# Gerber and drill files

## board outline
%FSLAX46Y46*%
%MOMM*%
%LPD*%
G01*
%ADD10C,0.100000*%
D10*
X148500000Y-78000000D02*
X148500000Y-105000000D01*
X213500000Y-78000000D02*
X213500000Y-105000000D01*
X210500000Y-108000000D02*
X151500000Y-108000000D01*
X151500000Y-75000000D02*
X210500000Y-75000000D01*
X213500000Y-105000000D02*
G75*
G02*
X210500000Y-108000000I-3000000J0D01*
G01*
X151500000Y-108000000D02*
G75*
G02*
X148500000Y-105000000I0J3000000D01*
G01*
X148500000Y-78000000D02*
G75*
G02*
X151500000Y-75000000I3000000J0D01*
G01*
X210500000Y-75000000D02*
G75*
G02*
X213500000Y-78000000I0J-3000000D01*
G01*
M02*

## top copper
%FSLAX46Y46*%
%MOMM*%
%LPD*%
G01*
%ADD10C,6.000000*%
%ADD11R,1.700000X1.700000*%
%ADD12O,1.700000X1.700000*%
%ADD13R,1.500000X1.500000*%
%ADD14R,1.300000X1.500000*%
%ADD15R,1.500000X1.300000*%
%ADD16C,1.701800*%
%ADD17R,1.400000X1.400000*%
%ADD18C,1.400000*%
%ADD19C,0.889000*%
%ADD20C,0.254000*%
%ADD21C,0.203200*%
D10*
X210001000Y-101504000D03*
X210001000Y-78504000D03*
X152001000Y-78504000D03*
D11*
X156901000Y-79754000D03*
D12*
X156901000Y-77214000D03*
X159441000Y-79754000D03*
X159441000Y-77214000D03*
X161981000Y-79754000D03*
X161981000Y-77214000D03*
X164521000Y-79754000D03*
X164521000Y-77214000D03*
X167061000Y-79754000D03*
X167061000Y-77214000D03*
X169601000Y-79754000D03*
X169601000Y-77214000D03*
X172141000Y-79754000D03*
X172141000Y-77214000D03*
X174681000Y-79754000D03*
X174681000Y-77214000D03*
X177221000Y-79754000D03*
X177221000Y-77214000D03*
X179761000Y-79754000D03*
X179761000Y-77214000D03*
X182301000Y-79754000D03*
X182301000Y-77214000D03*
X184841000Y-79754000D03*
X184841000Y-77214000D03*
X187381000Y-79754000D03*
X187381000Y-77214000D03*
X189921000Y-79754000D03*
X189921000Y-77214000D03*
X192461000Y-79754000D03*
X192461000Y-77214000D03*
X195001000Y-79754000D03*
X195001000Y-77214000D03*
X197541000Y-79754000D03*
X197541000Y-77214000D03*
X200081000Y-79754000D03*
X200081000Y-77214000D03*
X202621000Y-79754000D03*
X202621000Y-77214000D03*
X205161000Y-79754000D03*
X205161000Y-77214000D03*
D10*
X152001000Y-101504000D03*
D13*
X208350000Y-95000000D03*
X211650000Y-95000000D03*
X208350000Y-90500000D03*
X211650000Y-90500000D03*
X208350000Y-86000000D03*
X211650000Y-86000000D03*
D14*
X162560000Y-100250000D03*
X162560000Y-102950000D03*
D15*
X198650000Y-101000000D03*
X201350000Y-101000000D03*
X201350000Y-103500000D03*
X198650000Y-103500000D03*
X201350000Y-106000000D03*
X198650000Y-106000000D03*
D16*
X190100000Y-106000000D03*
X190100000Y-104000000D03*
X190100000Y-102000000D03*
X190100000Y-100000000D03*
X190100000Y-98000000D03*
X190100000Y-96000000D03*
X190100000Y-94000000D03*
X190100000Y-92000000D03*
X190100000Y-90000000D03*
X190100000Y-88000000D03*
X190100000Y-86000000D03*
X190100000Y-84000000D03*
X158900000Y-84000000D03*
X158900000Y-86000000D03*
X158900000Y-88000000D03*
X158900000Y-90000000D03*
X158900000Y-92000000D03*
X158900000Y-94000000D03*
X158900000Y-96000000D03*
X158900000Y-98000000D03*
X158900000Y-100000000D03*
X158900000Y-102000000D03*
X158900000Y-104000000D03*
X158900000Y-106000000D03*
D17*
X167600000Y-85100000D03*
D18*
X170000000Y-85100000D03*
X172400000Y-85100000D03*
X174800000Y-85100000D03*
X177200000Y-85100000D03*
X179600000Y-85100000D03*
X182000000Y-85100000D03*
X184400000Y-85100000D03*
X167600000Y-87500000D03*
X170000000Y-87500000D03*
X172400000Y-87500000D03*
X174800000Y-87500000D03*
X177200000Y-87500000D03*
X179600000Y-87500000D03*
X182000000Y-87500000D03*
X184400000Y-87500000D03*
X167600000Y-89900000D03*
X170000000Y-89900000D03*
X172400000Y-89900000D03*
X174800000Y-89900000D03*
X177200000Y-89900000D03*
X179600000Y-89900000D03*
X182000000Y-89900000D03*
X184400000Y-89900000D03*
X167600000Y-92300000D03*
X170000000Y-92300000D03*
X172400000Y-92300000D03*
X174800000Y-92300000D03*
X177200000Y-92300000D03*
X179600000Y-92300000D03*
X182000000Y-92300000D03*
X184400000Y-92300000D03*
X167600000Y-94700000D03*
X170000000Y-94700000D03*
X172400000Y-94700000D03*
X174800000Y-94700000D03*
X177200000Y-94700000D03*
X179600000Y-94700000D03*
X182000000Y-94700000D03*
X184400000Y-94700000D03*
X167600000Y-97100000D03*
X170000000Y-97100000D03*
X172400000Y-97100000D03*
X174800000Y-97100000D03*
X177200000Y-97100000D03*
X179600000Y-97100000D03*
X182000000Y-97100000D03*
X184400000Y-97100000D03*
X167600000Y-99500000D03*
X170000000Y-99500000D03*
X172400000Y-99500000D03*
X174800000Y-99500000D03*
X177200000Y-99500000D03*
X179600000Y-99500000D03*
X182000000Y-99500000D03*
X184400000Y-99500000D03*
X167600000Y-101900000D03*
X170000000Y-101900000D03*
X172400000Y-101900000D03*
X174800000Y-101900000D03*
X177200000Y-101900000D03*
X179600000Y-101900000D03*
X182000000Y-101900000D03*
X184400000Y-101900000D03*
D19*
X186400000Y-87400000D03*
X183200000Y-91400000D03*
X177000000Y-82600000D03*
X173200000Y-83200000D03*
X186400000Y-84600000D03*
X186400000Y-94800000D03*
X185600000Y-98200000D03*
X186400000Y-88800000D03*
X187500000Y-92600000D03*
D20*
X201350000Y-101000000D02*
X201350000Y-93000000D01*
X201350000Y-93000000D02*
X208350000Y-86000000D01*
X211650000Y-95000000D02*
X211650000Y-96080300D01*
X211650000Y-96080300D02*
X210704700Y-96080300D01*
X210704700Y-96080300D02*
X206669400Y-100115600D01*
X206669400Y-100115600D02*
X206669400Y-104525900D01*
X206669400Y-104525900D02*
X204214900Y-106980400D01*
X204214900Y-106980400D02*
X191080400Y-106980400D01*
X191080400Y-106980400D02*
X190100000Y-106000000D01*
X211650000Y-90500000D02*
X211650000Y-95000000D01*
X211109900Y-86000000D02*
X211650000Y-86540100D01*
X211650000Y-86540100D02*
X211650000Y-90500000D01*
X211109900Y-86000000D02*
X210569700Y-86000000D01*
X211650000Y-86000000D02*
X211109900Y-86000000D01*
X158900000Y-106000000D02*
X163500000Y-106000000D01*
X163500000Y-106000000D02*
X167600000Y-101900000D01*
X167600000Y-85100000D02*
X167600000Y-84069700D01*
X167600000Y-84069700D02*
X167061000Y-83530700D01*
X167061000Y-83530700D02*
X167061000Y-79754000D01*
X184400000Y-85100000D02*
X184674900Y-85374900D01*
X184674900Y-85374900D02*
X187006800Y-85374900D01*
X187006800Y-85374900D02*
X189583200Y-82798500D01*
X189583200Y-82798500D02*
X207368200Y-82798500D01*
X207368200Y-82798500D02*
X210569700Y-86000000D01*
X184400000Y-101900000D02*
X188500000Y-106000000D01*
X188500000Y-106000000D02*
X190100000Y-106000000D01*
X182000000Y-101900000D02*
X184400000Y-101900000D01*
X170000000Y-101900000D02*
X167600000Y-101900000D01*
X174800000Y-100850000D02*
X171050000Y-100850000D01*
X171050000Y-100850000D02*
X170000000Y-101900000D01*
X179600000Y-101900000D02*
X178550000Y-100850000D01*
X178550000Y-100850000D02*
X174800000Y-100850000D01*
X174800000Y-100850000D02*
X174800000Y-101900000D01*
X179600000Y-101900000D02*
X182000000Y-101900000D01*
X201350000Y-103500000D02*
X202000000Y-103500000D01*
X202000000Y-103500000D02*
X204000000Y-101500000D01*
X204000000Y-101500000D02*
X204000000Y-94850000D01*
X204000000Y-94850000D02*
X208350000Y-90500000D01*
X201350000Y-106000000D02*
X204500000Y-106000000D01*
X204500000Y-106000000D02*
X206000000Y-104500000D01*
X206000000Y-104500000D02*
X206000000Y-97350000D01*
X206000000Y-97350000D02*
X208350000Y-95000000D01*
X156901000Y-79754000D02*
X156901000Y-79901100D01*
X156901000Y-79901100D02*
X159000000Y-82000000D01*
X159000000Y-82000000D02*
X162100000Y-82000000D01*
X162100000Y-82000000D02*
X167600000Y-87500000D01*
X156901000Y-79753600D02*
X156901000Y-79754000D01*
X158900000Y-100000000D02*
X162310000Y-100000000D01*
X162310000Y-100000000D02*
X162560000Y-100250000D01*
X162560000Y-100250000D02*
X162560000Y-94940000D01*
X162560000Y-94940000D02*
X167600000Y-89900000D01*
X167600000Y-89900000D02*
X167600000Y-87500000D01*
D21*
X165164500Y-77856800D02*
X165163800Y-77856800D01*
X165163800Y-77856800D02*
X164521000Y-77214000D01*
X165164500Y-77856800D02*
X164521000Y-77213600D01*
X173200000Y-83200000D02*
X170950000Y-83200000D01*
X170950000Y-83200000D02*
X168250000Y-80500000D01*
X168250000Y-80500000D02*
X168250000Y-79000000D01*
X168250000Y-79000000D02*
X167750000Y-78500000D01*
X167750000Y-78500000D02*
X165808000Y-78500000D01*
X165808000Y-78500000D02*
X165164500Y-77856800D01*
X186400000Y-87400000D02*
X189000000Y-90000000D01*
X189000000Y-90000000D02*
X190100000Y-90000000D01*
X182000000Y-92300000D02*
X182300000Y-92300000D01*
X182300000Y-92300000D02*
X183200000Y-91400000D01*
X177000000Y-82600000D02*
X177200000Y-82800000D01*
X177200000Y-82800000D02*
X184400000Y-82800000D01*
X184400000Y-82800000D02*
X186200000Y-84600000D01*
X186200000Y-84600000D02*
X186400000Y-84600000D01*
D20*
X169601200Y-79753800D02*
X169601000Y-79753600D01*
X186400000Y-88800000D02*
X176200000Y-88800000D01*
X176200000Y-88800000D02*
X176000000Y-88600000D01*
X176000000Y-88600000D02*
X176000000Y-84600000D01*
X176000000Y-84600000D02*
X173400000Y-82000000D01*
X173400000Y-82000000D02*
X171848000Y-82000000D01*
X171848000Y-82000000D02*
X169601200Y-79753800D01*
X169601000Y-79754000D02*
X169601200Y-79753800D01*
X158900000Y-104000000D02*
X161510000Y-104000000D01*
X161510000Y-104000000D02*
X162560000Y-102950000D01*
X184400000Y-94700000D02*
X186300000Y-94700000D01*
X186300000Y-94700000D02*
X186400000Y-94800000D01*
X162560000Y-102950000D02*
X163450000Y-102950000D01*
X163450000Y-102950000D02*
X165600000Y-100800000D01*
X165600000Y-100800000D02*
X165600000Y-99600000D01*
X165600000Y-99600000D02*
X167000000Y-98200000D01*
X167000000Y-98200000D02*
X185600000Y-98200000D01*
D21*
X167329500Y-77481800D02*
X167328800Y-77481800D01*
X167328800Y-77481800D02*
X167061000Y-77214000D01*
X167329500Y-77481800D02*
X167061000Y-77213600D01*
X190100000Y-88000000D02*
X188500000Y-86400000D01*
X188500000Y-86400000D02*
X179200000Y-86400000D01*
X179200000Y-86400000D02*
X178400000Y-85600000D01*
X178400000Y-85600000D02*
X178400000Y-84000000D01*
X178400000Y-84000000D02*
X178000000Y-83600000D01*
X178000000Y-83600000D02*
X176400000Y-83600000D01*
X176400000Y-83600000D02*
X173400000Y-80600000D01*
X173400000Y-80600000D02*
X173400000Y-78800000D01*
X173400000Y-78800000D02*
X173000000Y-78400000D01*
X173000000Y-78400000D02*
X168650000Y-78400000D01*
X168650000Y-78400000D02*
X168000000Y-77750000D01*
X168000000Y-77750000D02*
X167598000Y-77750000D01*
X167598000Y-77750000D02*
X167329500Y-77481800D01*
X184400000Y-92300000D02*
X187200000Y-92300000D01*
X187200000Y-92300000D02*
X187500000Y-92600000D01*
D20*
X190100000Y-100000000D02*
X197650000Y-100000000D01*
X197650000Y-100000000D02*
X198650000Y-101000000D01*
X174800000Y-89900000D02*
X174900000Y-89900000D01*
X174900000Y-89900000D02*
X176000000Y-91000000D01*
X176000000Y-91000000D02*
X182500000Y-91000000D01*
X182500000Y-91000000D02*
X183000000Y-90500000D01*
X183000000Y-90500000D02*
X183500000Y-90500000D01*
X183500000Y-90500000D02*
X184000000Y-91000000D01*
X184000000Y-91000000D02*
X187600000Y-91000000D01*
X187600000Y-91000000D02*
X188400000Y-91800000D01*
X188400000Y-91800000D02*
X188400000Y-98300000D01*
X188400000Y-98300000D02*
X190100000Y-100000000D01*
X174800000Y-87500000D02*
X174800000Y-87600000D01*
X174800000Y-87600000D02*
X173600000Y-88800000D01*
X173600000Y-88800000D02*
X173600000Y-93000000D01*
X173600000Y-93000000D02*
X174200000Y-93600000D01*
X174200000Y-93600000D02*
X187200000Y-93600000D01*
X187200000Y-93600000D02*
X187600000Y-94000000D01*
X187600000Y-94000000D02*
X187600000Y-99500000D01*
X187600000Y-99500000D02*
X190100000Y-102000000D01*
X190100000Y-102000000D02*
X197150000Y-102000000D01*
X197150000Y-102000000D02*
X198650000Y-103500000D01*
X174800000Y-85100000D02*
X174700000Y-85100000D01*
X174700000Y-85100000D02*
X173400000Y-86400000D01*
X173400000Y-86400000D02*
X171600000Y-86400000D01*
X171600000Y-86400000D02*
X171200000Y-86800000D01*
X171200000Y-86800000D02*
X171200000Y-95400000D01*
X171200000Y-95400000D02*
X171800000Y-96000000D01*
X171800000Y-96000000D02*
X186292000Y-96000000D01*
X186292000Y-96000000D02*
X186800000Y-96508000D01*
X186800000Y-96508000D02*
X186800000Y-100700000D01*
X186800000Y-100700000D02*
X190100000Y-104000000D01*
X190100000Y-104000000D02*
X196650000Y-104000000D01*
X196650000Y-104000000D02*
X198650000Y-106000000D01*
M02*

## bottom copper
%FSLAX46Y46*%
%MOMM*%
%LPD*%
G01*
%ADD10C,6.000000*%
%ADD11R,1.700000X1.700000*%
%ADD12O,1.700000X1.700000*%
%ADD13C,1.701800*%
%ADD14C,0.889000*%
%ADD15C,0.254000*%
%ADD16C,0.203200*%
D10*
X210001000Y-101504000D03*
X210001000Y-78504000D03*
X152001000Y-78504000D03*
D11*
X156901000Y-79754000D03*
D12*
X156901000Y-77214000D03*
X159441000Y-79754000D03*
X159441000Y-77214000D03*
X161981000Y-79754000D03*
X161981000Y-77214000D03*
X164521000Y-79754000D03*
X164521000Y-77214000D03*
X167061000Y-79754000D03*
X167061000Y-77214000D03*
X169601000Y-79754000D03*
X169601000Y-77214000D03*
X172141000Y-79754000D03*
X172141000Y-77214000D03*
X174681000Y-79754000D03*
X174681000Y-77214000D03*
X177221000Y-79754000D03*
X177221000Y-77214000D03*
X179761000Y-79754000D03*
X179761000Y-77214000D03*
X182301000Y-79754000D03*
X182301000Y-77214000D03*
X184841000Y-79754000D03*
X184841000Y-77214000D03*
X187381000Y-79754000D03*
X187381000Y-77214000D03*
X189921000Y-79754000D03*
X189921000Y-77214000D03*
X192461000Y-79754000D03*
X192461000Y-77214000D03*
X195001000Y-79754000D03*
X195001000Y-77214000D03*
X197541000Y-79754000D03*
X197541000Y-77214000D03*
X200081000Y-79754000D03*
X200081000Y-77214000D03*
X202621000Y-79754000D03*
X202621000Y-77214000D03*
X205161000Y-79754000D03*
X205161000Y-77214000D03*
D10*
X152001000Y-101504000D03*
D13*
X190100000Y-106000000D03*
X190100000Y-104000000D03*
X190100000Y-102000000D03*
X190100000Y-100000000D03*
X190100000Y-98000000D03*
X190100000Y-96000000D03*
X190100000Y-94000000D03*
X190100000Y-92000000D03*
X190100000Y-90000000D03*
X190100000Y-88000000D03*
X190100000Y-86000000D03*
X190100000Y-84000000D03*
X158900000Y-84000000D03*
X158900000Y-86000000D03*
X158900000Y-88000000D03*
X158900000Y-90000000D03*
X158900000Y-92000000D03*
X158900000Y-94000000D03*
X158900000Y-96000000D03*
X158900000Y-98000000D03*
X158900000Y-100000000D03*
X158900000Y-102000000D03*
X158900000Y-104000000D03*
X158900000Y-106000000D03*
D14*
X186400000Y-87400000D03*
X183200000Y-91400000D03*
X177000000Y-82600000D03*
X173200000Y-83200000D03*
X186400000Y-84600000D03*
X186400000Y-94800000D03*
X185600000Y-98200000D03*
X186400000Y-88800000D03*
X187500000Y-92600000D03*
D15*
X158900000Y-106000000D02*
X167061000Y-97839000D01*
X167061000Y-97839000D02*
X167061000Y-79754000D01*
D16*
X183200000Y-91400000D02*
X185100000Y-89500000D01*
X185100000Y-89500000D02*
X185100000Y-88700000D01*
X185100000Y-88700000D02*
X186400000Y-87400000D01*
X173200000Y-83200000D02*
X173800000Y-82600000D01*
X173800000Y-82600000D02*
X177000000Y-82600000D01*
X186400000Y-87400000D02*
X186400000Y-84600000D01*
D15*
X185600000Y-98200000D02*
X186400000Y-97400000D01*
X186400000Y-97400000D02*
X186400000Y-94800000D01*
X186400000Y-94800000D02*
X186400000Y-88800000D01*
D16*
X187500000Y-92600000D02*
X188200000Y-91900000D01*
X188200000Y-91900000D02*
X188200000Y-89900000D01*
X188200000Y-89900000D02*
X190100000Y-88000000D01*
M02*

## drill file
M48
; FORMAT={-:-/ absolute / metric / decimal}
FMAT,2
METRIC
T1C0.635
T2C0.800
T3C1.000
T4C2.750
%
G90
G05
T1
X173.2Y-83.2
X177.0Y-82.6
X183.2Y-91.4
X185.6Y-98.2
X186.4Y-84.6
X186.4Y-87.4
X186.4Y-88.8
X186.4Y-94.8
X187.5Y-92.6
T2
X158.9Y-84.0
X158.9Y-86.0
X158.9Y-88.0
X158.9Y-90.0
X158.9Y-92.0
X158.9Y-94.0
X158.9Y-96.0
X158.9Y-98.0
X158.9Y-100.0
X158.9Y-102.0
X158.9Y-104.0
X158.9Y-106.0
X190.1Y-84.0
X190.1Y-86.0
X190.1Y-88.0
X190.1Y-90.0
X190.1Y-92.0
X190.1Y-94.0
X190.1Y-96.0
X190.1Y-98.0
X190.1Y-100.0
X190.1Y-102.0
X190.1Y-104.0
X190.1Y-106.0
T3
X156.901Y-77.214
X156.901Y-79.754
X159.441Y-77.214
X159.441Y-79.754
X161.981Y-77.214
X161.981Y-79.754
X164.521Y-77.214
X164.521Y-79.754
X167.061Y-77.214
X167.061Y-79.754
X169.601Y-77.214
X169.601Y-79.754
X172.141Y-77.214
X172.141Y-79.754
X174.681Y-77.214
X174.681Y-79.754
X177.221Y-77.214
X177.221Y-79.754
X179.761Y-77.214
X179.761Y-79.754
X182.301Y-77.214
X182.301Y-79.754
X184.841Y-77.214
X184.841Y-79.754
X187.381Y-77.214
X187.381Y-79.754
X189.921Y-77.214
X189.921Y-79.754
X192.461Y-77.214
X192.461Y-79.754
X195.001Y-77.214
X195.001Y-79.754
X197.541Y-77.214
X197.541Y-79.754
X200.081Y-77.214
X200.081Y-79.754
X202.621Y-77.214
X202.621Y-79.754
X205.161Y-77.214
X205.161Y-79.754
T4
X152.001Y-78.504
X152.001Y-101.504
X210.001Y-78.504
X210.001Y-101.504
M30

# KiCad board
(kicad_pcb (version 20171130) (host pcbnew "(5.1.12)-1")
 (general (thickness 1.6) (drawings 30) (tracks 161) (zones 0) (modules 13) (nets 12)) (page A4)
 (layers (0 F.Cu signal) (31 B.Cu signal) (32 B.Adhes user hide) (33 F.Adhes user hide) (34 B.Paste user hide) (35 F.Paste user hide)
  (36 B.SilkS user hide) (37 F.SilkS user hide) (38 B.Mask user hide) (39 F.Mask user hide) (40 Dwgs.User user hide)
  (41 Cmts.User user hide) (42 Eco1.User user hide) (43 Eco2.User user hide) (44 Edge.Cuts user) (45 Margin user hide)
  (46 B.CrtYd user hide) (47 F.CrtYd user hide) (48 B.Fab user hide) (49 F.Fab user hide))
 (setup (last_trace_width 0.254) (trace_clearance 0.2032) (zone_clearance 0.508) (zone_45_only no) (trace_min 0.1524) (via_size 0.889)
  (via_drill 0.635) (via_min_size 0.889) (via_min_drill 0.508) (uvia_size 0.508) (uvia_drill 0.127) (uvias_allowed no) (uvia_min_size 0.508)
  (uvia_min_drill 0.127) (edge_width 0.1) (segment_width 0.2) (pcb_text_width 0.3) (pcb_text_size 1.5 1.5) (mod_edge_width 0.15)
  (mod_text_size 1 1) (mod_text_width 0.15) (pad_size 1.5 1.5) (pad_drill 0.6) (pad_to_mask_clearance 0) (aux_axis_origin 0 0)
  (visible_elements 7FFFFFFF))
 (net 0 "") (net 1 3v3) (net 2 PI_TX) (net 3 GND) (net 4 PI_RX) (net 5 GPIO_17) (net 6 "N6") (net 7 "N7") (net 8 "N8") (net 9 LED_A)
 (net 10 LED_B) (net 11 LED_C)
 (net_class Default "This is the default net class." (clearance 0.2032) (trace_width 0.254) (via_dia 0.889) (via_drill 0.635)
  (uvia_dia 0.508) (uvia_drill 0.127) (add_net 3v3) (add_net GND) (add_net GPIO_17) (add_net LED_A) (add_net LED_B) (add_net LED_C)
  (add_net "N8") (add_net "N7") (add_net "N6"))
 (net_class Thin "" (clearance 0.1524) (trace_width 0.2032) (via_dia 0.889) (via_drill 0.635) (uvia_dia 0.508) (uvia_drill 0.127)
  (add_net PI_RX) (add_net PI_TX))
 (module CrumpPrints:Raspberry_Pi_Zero (layer F.Cu) (at 148.501 105.004)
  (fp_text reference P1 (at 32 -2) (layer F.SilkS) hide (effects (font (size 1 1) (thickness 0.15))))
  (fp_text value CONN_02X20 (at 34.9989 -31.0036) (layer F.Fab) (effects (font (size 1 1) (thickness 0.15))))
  (pad "" np_thru_hole circle (at 61.5 -3.5) (size 6 6) (drill 2.75) (layers *.Cu *.Mask F.SilkS))
  (pad "" np_thru_hole circle (at 61.5 -26.5) (size 6 6) (drill 2.75) (layers *.Cu *.Mask F.SilkS))
  (pad "" np_thru_hole circle (at 3.5 -26.5) (size 6 6) (drill 2.75) (layers *.Cu *.Mask F.SilkS))
  (pad 1 thru_hole rect (at 8.4 -25.25 90) (size 1.7 1.7) (drill 1) (layers *.Cu *.Mask) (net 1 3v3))
  (pad 2 thru_hole oval (at 8.4 -27.79 90) (size 1.7 1.7) (drill 1) (layers *.Cu *.Mask))
  (pad 3 thru_hole oval (at 10.94 -25.25 90) (size 1.7 1.7) (drill 1) (layers *.Cu *.Mask))
  (pad 4 thru_hole oval (at 10.94 -27.79 90) (size 1.7 1.7) (drill 1) (layers *.Cu *.Mask))
  (pad 5 thru_hole oval (at 13.48 -25.25 90) (size 1.7 1.7) (drill 1) (layers *.Cu *.Mask))
  (pad 6 thru_hole oval (at 13.48 -27.79 90) (size 1.7 1.7) (drill 1) (layers *.Cu *.Mask))
  (pad 7 thru_hole oval (at 16.02 -25.25 90) (size 1.7 1.7) (drill 1) (layers *.Cu *.Mask))
  (pad 8 thru_hole oval (at 16.02 -27.79 90) (size 1.7 1.7) (drill 1) (layers *.Cu *.Mask) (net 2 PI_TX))
  (pad 9 thru_hole oval (at 18.56 -25.25 90) (size 1.7 1.7) (drill 1) (layers *.Cu *.Mask) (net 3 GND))
  (pad 10 thru_hole oval (at 18.56 -27.79 90) (size 1.7 1.7) (drill 1) (layers *.Cu *.Mask) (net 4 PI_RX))
  (pad 11 thru_hole oval (at 21.1 -25.25 90) (size 1.7 1.7) (drill 1) (layers *.Cu *.Mask) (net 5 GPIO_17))
  (pad 12 thru_hole oval (at 21.1 -27.79 90) (size 1.7 1.7) (drill 1) (layers *.Cu *.Mask))
  (pad 13 thru_hole oval (at 23.64 -25.25 90) (size 1.7 1.7) (drill 1) (layers *.Cu *.Mask))
  (pad 14 thru_hole oval (at 23.64 -27.79 90) (size 1.7 1.7) (drill 1) (layers *.Cu *.Mask))
  (pad 15 thru_hole oval (at 26.18 -25.25 90) (size 1.7 1.7) (drill 1) (layers *.Cu *.Mask))
  (pad 16 thru_hole oval (at 26.18 -27.79 90) (size 1.7 1.7) (drill 1) (layers *.Cu *.Mask))
  (pad 17 thru_hole oval (at 28.72 -25.25 90) (size 1.7 1.7) (drill 1) (layers *.Cu *.Mask))
  (pad 18 thru_hole oval (at 28.72 -27.79 90) (size 1.7 1.7) (drill 1) (layers *.Cu *.Mask))
  (pad 19 thru_hole oval (at 31.26 -25.25 90) (size 1.7 1.7) (drill 1) (layers *.Cu *.Mask))
  (pad 20 thru_hole oval (at 31.26 -27.79 90) (size 1.7 1.7) (drill 1) (layers *.Cu *.Mask))
  (pad 21 thru_hole oval (at 33.8 -25.25 90) (size 1.7 1.7) (drill 1) (layers *.Cu *.Mask))
  (pad 22 thru_hole oval (at 33.8 -27.79 90) (size 1.7 1.7) (drill 1) (layers *.Cu *.Mask))
  (pad 23 thru_hole oval (at 36.34 -25.25 90) (size 1.7 1.7) (drill 1) (layers *.Cu *.Mask))
  (pad 24 thru_hole oval (at 36.34 -27.79 90) (size 1.7 1.7) (drill 1) (layers *.Cu *.Mask))
  (pad 25 thru_hole oval (at 38.88 -25.25 90) (size 1.7 1.7) (drill 1) (layers *.Cu *.Mask))
  (pad 26 thru_hole oval (at 38.88 -27.79 90) (size 1.7 1.7) (drill 1) (layers *.Cu *.Mask))
  (pad 27 thru_hole oval (at 41.42 -25.25 90) (size 1.7 1.7) (drill 1) (layers *.Cu *.Mask))
  (pad 28 thru_hole oval (at 41.42 -27.79 90) (size 1.7 1.7) (drill 1) (layers *.Cu *.Mask))
  (pad 29 thru_hole oval (at 43.96 -25.25 90) (size 1.7 1.7) (drill 1) (layers *.Cu *.Mask))
  (pad 30 thru_hole oval (at 43.96 -27.79 90) (size 1.7 1.7) (drill 1) (layers *.Cu *.Mask))
  (pad 31 thru_hole oval (at 46.5 -25.25 90) (size 1.7 1.7) (drill 1) (layers *.Cu *.Mask))
  (pad 32 thru_hole oval (at 46.5 -27.79 90) (size 1.7 1.7) (drill 1) (layers *.Cu *.Mask))
  (pad 33 thru_hole oval (at 49.04 -25.25 90) (size 1.7 1.7) (drill 1) (layers *.Cu *.Mask))
  (pad 34 thru_hole oval (at 49.04 -27.79 90) (size 1.7 1.7) (drill 1) (layers *.Cu *.Mask))
  (pad 35 thru_hole oval (at 51.58 -25.25 90) (size 1.7 1.7) (drill 1) (layers *.Cu *.Mask))
  (pad 36 thru_hole oval (at 51.58 -27.79 90) (size 1.7 1.7) (drill 1) (layers *.Cu *.Mask))
  (pad 37 thru_hole oval (at 54.12 -25.25 90) (size 1.7 1.7) (drill 1) (layers *.Cu *.Mask))
  (pad 38 thru_hole oval (at 54.12 -27.79 90) (size 1.7 1.7) (drill 1) (layers *.Cu *.Mask))
  (pad 39 thru_hole oval (at 56.66 -25.25 90) (size 1.7 1.7) (drill 1) (layers *.Cu *.Mask))
  (pad 40 thru_hole oval (at 56.66 -27.79 90) (size 1.7 1.7) (drill 1) (layers *.Cu *.Mask))
  (pad "" np_thru_hole circle (at 3.5 -3.5) (size 6 6) (drill 2.75) (layers *.Cu *.Mask F.SilkS)))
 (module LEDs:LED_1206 (layer F.Cu) (at 210 95 180)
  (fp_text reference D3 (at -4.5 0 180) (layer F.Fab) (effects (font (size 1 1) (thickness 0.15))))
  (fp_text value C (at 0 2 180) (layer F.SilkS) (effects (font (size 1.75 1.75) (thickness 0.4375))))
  (pad 2 smd rect (at 1.65 0) (size 1.5 1.5) (layers F.Cu F.Paste F.Mask) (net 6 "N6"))
  (pad 1 smd rect (at -1.65 0) (size 1.5 1.5) (layers F.Cu F.Paste F.Mask) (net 3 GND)))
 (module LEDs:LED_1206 (layer F.Cu) (at 210 90.5 180)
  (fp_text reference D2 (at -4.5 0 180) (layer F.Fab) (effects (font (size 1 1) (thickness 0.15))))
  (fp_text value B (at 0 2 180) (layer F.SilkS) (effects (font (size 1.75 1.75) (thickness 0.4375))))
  (pad 2 smd rect (at 1.65 0) (size 1.5 1.5) (layers F.Cu F.Paste F.Mask) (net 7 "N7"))
  (pad 1 smd rect (at -1.65 0) (size 1.5 1.5) (layers F.Cu F.Paste F.Mask) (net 3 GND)))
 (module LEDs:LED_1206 (layer F.Cu) (at 210 86 180)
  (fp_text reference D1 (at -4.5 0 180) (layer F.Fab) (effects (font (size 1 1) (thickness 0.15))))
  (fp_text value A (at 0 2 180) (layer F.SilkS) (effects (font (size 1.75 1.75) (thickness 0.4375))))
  (pad 2 smd rect (at 1.65 0) (size 1.5 1.5) (layers F.Cu F.Paste F.Mask) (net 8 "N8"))
  (pad 1 smd rect (at -1.65 0) (size 1.5 1.5) (layers F.Cu F.Paste F.Mask) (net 3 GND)))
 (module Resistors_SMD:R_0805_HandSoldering (layer F.Cu) (at 162.56 101.6 270)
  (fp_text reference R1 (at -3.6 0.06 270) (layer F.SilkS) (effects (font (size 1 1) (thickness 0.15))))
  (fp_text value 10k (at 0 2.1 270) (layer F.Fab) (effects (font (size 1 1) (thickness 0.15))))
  (pad 1 smd rect (at -1.35 0 270) (size 1.5 1.3) (layers F.Cu F.Paste F.Mask) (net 1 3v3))
  (pad 2 smd rect (at 1.35 0 270) (size 1.5 1.3) (layers F.Cu F.Paste F.Mask) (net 5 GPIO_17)))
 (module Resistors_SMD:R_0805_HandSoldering (layer F.Cu) (at 200 101)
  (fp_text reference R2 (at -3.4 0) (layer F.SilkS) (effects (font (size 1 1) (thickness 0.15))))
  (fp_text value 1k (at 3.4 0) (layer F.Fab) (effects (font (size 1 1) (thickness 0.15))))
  (pad 1 smd rect (at -1.35 0) (size 1.5 1.3) (layers F.Cu F.Paste F.Mask) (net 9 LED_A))
  (pad 2 smd rect (at 1.35 0) (size 1.5 1.3) (layers F.Cu F.Paste F.Mask) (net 8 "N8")))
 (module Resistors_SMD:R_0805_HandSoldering (layer F.Cu) (at 200 103.5 180)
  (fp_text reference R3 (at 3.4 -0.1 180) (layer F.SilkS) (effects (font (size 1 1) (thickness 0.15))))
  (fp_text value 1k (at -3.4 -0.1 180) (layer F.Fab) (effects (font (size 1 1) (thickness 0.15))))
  (pad 1 smd rect (at -1.35 0 180) (size 1.5 1.3) (layers F.Cu F.Paste F.Mask) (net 7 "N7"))
  (pad 2 smd rect (at 1.35 0 180) (size 1.5 1.3) (layers F.Cu F.Paste F.Mask) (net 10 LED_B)))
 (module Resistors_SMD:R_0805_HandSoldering (layer F.Cu) (at 200 106 180)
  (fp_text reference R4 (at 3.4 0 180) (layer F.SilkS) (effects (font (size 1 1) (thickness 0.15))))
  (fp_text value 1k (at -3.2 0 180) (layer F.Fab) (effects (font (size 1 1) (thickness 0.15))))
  (pad 1 smd rect (at -1.35 0 180) (size 1.5 1.3) (layers F.Cu F.Paste F.Mask) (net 6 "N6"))
  (pad 2 smd rect (at 1.35 0 180) (size 1.5 1.3) (layers F.Cu F.Paste F.Mask) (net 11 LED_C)))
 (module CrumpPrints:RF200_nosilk (layer F.Cu) (at 174.5 95 180)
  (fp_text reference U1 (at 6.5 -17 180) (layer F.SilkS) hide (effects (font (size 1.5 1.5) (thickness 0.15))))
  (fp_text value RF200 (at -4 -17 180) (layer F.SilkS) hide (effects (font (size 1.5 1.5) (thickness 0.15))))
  (pad 1 thru_hole circle (at -15.6 -11 180) (size 1.7018 1.7018) (drill 0.800001) (layers *.Cu *.Mask) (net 3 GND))
  (pad 2 thru_hole circle (at -15.6 -9 180) (size 1.7018 1.7018) (drill 0.800001) (layers *.Cu *.Mask) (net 11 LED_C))
  (pad 3 thru_hole circle (at -15.6 -7 180) (size 1.7018 1.7018) (drill 0.800001) (layers *.Cu *.Mask) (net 10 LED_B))
  (pad 4 thru_hole circle (at -15.6 -5 180) (size 1.7018 1.7018) (drill 0.800001) (layers *.Cu *.Mask) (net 9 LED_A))
  (pad 5 thru_hole circle (at -15.6 -3 180) (size 1.7018 1.7018) (drill 0.800001) (layers *.Cu *.Mask))
  (pad 6 thru_hole circle (at -15.6 -1 180) (size 1.7018 1.7018) (drill 0.800001) (layers *.Cu *.Mask))
  (pad 7 thru_hole circle (at -15.6 1 180) (size 1.7018 1.7018) (drill 0.800001) (layers *.Cu *.Mask))
  (pad 8 thru_hole circle (at -15.6 3 180) (size 1.7018 1.7018) (drill 0.800001) (layers *.Cu *.Mask))
  (pad 9 thru_hole circle (at -15.6 5 180) (size 1.7018 1.7018) (drill 0.800001) (layers *.Cu *.Mask) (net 2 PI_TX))
  (pad 10 thru_hole circle (at -15.6 7 180) (size 1.7018 1.7018) (drill 0.800001) (layers *.Cu *.Mask) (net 4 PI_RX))
  (pad 11 thru_hole circle (at -15.6 9 180) (size 1.7018 1.7018) (drill 0.800001) (layers *.Cu *.Mask))
  (pad 12 thru_hole circle (at -15.6 11 180) (size 1.7018 1.7018) (drill 0.800001) (layers *.Cu *.Mask))
  (pad 13 thru_hole circle (at 15.6 11 180) (size 1.7018 1.7018) (drill 0.800001) (layers *.Cu *.Mask))
  (pad 14 thru_hole circle (at 15.6 9 180) (size 1.7018 1.7018) (drill 0.800001) (layers *.Cu *.Mask))
  (pad 15 thru_hole circle (at 15.6 7 180) (size 1.7018 1.7018) (drill 0.800001) (layers *.Cu *.Mask))
  (pad 16 thru_hole circle (at 15.6 5 180) (size 1.7018 1.7018) (drill 0.800001) (layers *.Cu *.Mask))
  (pad 17 thru_hole circle (at 15.6 3 180) (size 1.7018 1.7018) (drill 0.800001) (layers *.Cu *.Mask))
  (pad 18 thru_hole circle (at 15.6 1 180) (size 1.7018 1.7018) (drill 0.800001) (layers *.Cu *.Mask))
  (pad 19 thru_hole circle (at 15.6 -1 180) (size 1.7018 1.7018) (drill 0.800001) (layers *.Cu *.Mask))
  (pad 20 thru_hole circle (at 15.6 -3 180) (size 1.7018 1.7018) (drill 0.800001) (layers *.Cu *.Mask))
  (pad 21 thru_hole circle (at 15.6 -5 180) (size 1.7018 1.7018) (drill 0.800001) (layers *.Cu *.Mask) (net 1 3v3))
  (pad 22 thru_hole circle (at 15.6 -7 180) (size 1.7018 1.7018) (drill 0.800001) (layers *.Cu *.Mask))
  (pad 23 thru_hole circle (at 15.6 -9 180) (size 1.7018 1.7018) (drill 0.800001) (layers *.Cu *.Mask) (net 5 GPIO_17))
  (pad 24 thru_hole circle (at 15.6 -11 180) (size 1.7018 1.7018) (drill 0.800001) (layers *.Cu *.Mask) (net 3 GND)))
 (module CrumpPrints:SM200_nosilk (layer F.Cu) (at 176 93.5 180)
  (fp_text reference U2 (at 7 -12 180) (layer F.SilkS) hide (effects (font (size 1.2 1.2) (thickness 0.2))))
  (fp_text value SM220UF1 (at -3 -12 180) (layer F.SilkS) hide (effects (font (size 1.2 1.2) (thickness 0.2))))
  (pad A1 smd rect (at 8.4 8.4 270) (size 1.4 1.4) (layers F.Cu F.Paste F.Mask) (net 3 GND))
  (pad B1 smd circle (at 6 8.4 270) (size 1.4 1.4) (layers F.Cu F.Paste F.Mask))
  (pad C1 smd circle (at 3.6 8.4 270) (size 1.4 1.4) (layers F.Cu F.Paste F.Mask))
  (pad D1 smd circle (at 1.2 8.4 270) (size 1.4 1.4) (layers F.Cu F.Paste F.Mask) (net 11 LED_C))
  (pad E1 smd circle (at -1.2 8.4 270) (size 1.4 1.4) (layers F.Cu F.Paste F.Mask))
  (pad F1 smd circle (at -3.6 8.4 270) (size 1.4 1.4) (layers F.Cu F.Paste F.Mask))
  (pad G1 smd circle (at -6 8.4 270) (size 1.4 1.4) (layers F.Cu F.Paste F.Mask))
  (pad H1 smd circle (at -8.4 8.4 270) (size 1.4 1.4) (layers F.Cu F.Paste F.Mask) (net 3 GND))
  (pad A2 smd circle (at 8.4 6 270) (size 1.4 1.4) (layers F.Cu F.Paste F.Mask) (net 1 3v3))
  (pad B2 smd circle (at 6 6 270) (size 1.4 1.4) (layers F.Cu F.Paste F.Mask))
  (pad C2 smd circle (at 3.6 6 270) (size 1.4 1.4) (layers F.Cu F.Paste F.Mask))
  (pad D2 smd circle (at 1.2 6 270) (size 1.4 1.4) (layers F.Cu F.Paste F.Mask) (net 10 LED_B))
  (pad E2 smd circle (at -1.2 6 270) (size 1.4 1.4) (layers F.Cu F.Paste F.Mask))
  (pad F2 smd circle (at -3.6 6 270) (size 1.4 1.4) (layers F.Cu F.Paste F.Mask))
  (pad G2 smd circle (at -6 6 270) (size 1.4 1.4) (layers F.Cu F.Paste F.Mask))
  (pad H2 smd circle (at -8.4 6 270) (size 1.4 1.4) (layers F.Cu F.Paste F.Mask))
  (pad A3 smd circle (at 8.4 3.6 270) (size 1.4 1.4) (layers F.Cu F.Paste F.Mask) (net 1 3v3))
  (pad B3 smd circle (at 6 3.6 270) (size 1.4 1.4) (layers F.Cu F.Paste F.Mask))
  (pad C3 smd circle (at 3.6 3.6 270) (size 1.4 1.4) (layers F.Cu F.Paste F.Mask))
  (pad D3 smd circle (at 1.2 3.6 270) (size 1.4 1.4) (layers F.Cu F.Paste F.Mask) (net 9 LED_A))
  (pad E3 smd circle (at -1.2 3.6 270) (size 1.4 1.4) (layers F.Cu F.Paste F.Mask))
  (pad F3 smd circle (at -3.6 3.6 270) (size 1.4 1.4) (layers F.Cu F.Paste F.Mask))
  (pad G3 smd circle (at -6 3.6 270) (size 1.4 1.4) (layers F.Cu F.Paste F.Mask))
  (pad H3 smd circle (at -8.4 3.6 270) (size 1.4 1.4) (layers F.Cu F.Paste F.Mask))
  (pad A4 smd circle (at 8.4 1.2 270) (size 1.4 1.4) (layers F.Cu F.Paste F.Mask))
  (pad B4 smd circle (at 6 1.2 270) (size 1.4 1.4) (layers F.Cu F.Paste F.Mask))
  (pad C4 smd circle (at 3.6 1.2 270) (size 1.4 1.4) (layers F.Cu F.Paste F.Mask))
  (pad D4 smd circle (at 1.2 1.2 270) (size 1.4 1.4) (layers F.Cu F.Paste F.Mask))
  (pad E4 smd circle (at -1.2 1.2 270) (size 1.4 1.4) (layers F.Cu F.Paste F.Mask))
  (pad F4 smd circle (at -3.6 1.2 270) (size 1.4 1.4) (layers F.Cu F.Paste F.Mask))
  (pad G4 smd circle (at -6 1.2 270) (size 1.4 1.4) (layers F.Cu F.Paste F.Mask) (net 2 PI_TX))
  (pad H4 smd circle (at -8.4 1.2 270) (size 1.4 1.4) (layers F.Cu F.Paste F.Mask) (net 4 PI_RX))
  (pad A5 smd circle (at 8.4 -1.2 270) (size 1.4 1.4) (layers F.Cu F.Paste F.Mask))
  (pad B5 smd circle (at 6 -1.2 270) (size 1.4 1.4) (layers F.Cu F.Paste F.Mask))
  (pad C5 smd circle (at 3.6 -1.2 270) (size 1.4 1.4) (layers F.Cu F.Paste F.Mask))
  (pad D5 smd circle (at 1.2 -1.2 270) (size 1.4 1.4) (layers F.Cu F.Paste F.Mask))
  (pad E5 smd circle (at -1.2 -1.2 270) (size 1.4 1.4) (layers F.Cu F.Paste F.Mask))
  (pad F5 smd circle (at -3.6 -1.2 270) (size 1.4 1.4) (layers F.Cu F.Paste F.Mask))
  (pad G5 smd circle (at -6 -1.2 270) (size 1.4 1.4) (layers F.Cu F.Paste F.Mask))
  (pad H5 smd circle (at -8.4 -1.2 270) (size 1.4 1.4) (layers F.Cu F.Paste F.Mask) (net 5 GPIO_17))
  (pad A6 smd circle (at 8.4 -3.6 270) (size 1.4 1.4) (layers F.Cu F.Paste F.Mask))
  (pad B6 smd circle (at 6 -3.6 270) (size 1.4 1.4) (layers F.Cu F.Paste F.Mask))
  (pad C6 smd circle (at 3.6 -3.6 270) (size 1.4 1.4) (layers F.Cu F.Paste F.Mask))
  (pad D6 smd circle (at 1.2 -3.6 270) (size 1.4 1.4) (layers F.Cu F.Paste F.Mask))
  (pad E6 smd circle (at -1.2 -3.6 270) (size 1.4 1.4) (layers F.Cu F.Paste F.Mask))
  (pad F6 smd circle (at -3.6 -3.6 270) (size 1.4 1.4) (layers F.Cu F.Paste F.Mask))
  (pad G6 smd circle (at -6 -3.6 270) (size 1.4 1.4) (layers F.Cu F.Paste F.Mask))
  (pad H6 smd circle (at -8.4 -3.6 270) (size 1.4 1.4) (layers F.Cu F.Paste F.Mask))
  (pad A7 smd circle (at 8.4 -6 270) (size 1.4 1.4) (layers F.Cu F.Paste F.Mask))
  (pad B7 smd circle (at 6 -6 270) (size 1.4 1.4) (layers F.Cu F.Paste F.Mask))
  (pad C7 smd circle (at 3.6 -6 270) (size 1.4 1.4) (layers F.Cu F.Paste F.Mask))
  (pad D7 smd circle (at 1.2 -6 270) (size 1.4 1.4) (layers F.Cu F.Paste F.Mask))
  (pad E7 smd circle (at -1.2 -6 270) (size 1.4 1.4) (layers F.Cu F.Paste F.Mask))
  (pad F7 smd circle (at -3.6 -6 270) (size 1.4 1.4) (layers F.Cu F.Paste F.Mask))
  (pad G7 smd circle (at -6 -6 270) (size 1.4 1.4) (layers F.Cu F.Paste F.Mask))
  (pad H7 smd circle (at -8.4 -6 270) (size 1.4 1.4) (layers F.Cu F.Paste F.Mask))
  (pad A8 smd circle (at 8.4 -8.4 270) (size 1.4 1.4) (layers F.Cu F.Paste F.Mask) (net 3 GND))
  (pad B8 smd circle (at 6 -8.4 270) (size 1.4 1.4) (layers F.Cu F.Paste F.Mask) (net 3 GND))
  (pad C8 smd circle (at 3.6 -8.4 270) (size 1.4 1.4) (layers F.Cu F.Paste F.Mask))
  (pad D8 smd circle (at 1.2 -8.4 270) (size 1.4 1.4) (layers F.Cu F.Paste F.Mask) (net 3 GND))
  (pad E8 smd circle (at -1.2 -8.4 270) (size 1.4 1.4) (layers F.Cu F.Paste F.Mask))
  (pad F8 smd circle (at -3.6 -8.4 270) (size 1.4 1.4) (layers F.Cu F.Paste F.Mask) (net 3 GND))
  (pad G8 smd circle (at -6 -8.4 270) (size 1.4 1.4) (layers F.Cu F.Paste F.Mask) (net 3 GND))
  (pad H8 smd circle (at -8.4 -8.4 270) (size 1.4 1.4) (layers F.Cu F.Paste F.Mask) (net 3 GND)))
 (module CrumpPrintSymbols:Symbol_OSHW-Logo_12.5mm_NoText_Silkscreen (layer B.Cu) (at 202 87 180)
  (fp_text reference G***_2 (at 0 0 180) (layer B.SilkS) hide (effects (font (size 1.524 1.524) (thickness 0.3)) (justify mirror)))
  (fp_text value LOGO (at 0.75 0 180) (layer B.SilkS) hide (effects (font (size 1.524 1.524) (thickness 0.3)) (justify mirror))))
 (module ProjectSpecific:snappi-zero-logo (layer F.Cu) (at 199.5 89)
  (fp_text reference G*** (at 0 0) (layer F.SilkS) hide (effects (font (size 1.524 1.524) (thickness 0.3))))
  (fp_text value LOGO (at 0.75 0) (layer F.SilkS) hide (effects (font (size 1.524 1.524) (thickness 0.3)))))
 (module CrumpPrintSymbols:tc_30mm (layer F.Cu) (at 152.5 85.5)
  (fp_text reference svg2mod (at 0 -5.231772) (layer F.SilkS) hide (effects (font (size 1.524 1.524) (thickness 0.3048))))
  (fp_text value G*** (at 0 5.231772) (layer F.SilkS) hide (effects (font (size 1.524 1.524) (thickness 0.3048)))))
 (gr_line (start 148.5 78) (end 148.5 105) (angle 90) (layer Edge.Cuts) (width 0.1))
 (gr_line (start 213.5 78) (end 213.5 105) (angle 90) (layer Edge.Cuts) (width 0.1))
 (gr_line (start 210.5 108) (end 151.5 108) (angle 90) (layer Edge.Cuts) (width 0.1))
 (gr_line (start 151.5 75) (end 210.5 75) (angle 90) (layer Edge.Cuts) (width 0.1))
 (gr_arc (start 210.5 105) (end 213.5 105) (angle 90) (layer Edge.Cuts) (width 0.1))
 (gr_arc (start 151.5 105) (end 151.5 108) (angle 90) (layer Edge.Cuts) (width 0.1))
 (gr_arc (start 151.5 78) (end 148.5 78) (angle 90) (layer Edge.Cuts) (width 0.1))
 (gr_arc (start 210.5 78) (end 210.5 75) (angle 90) (layer Edge.Cuts) (width 0.1))
 (segment (start 201.35 101) (end 201.35 93) (width 0.254) (layer F.Cu) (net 8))
 (segment (start 201.35 93) (end 208.35 86) (width 0.254) (layer F.Cu) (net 8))
 (segment (start 211.65 95) (end 211.65 96.0803) (width 0.254) (layer F.Cu) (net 3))
 (segment (start 211.65 96.0803) (end 210.7047 96.0803) (width 0.254) (layer F.Cu) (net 3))
 (segment (start 210.7047 96.0803) (end 206.6694 100.1156) (width 0.254) (layer F.Cu) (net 3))
 (segment (start 206.6694 100.1156) (end 206.6694 104.5259) (width 0.254) (layer F.Cu) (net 3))
 (segment (start 206.6694 104.5259) (end 204.2149 106.9804) (width 0.254) (layer F.Cu) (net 3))
 (segment (start 204.2149 106.9804) (end 191.0804 106.9804) (width 0.254) (layer F.Cu) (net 3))
 (segment (start 191.0804 106.9804) (end 190.1 106) (width 0.254) (layer F.Cu) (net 3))
 (segment (start 211.65 90.5) (end 211.65 95) (width 0.254) (layer F.Cu) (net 3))
 (segment (start 211.1099 86) (end 211.65 86.5401) (width 0.254) (layer F.Cu) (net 3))
 (segment (start 211.65 86.5401) (end 211.65 90.5) (width 0.254) (layer F.Cu) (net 3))
 (segment (start 211.1099 86) (end 210.5697 86) (width 0.254) (layer F.Cu) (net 3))
 (segment (start 211.65 86) (end 211.1099 86) (width 0.254) (layer F.Cu) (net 3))
 (segment (start 158.9 106) (end 167.061 97.839) (width 0.254) (layer B.Cu) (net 3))
 (segment (start 167.061 97.839) (end 167.061 79.754) (width 0.254) (layer B.Cu) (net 3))
 (segment (start 158.9 106) (end 163.5 106) (width 0.254) (layer F.Cu) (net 3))
 (segment (start 163.5 106) (end 167.6 101.9) (width 0.254) (layer F.Cu) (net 3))
 (segment (start 167.6 85.1) (end 167.6 84.0697) (width 0.254) (layer F.Cu) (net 3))
 (segment (start 167.6 84.0697) (end 167.061 83.5307) (width 0.254) (layer F.Cu) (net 3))
 (segment (start 167.061 83.5307) (end 167.061 79.754) (width 0.254) (layer F.Cu) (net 3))
 (segment (start 184.4 85.1) (end 184.6749 85.3749) (width 0.254) (layer F.Cu) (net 3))
 (segment (start 184.6749 85.3749) (end 187.0068 85.3749) (width 0.254) (layer F.Cu) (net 3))
 (segment (start 187.0068 85.3749) (end 189.5832 82.7985) (width 0.254) (layer F.Cu) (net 3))
 (segment (start 189.5832 82.7985) (end 207.3682 82.7985) (width 0.254) (layer F.Cu) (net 3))
 (segment (start 207.3682 82.7985) (end 210.5697 86) (width 0.254) (layer F.Cu) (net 3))
 (segment (start 184.4 101.9) (end 188.5 106) (width 0.254) (layer F.Cu) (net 3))
 (segment (start 188.5 106) (end 190.1 106) (width 0.254) (layer F.Cu) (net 3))
 (segment (start 182 101.9) (end 184.4 101.9) (width 0.254) (layer F.Cu) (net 3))
 (segment (start 170 101.9) (end 167.6 101.9) (width 0.254) (layer F.Cu) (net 3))
 (segment (start 174.8 100.85) (end 171.05 100.85) (width 0.254) (layer F.Cu) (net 3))
 (segment (start 171.05 100.85) (end 170 101.9) (width 0.254) (layer F.Cu) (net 3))
 (segment (start 179.6 101.9) (end 178.55 100.85) (width 0.254) (layer F.Cu) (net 3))
 (segment (start 178.55 100.85) (end 174.8 100.85) (width 0.254) (layer F.Cu) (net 3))
 (segment (start 174.8 100.85) (end 174.8 101.9) (width 0.254) (layer F.Cu) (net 3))
 (segment (start 179.6 101.9) (end 182 101.9) (width 0.254) (layer F.Cu) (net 3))
 (segment (start 201.35 103.5) (end 202 103.5) (width 0.254) (layer F.Cu) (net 7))
 (segment (start 202 103.5) (end 204 101.5) (width 0.254) (layer F.Cu) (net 7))
 (segment (start 204 101.5) (end 204 94.85) (width 0.254) (layer F.Cu) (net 7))
 (segment (start 204 94.85) (end 208.35 90.5) (width 0.254) (layer F.Cu) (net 7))
 (segment (start 201.35 106) (end 204.5 106) (width 0.254) (layer F.Cu) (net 6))
 (segment (start 204.5 106) (end 206 104.5) (width 0.254) (layer F.Cu) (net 6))
 (segment (start 206 104.5) (end 206 97.35) (width 0.254) (layer F.Cu) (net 6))
 (segment (start 206 97.35) (end 208.35 95) (width 0.254) (layer F.Cu) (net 6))
 (segment (start 156.901 79.754) (end 156.901 79.9011) (width 0.254) (layer F.Cu) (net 1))
 (segment (start 156.901 79.9011) (end 159 82) (width 0.254) (layer F.Cu) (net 1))
 (segment (start 159 82) (end 162.1 82) (width 0.254) (layer F.Cu) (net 1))
 (segment (start 162.1 82) (end 167.6 87.5) (width 0.254) (layer F.Cu) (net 1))
 (segment (start 156.901 79.7536) (end 156.901 79.754) (width 0.254) (layer F.Cu) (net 1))
 (segment (start 158.9 100) (end 162.31 100) (width 0.254) (layer F.Cu) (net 1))
 (segment (start 162.31 100) (end 162.56 100.25) (width 0.254) (layer F.Cu) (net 1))
 (segment (start 162.56 100.25) (end 162.56 94.94) (width 0.254) (layer F.Cu) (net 1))
 (segment (start 162.56 94.94) (end 167.6 89.9) (width 0.254) (layer F.Cu) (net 1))
 (segment (start 167.6 89.9) (end 167.6 87.5) (width 0.254) (layer F.Cu) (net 1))
 (segment (start 165.1645 77.8568) (end 165.1638 77.8568) (width 0.2032) (layer F.Cu) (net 2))
 (segment (start 165.1638 77.8568) (end 164.521 77.214) (width 0.2032) (layer F.Cu) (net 2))
 (segment (start 165.1645 77.8568) (end 164.521 77.2136) (width 0.2032) (layer F.Cu) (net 2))
 (segment (start 173.2 83.2) (end 170.95 83.2) (width 0.2032) (layer F.Cu) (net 2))
 (segment (start 170.95 83.2) (end 168.25 80.5) (width 0.2032) (layer F.Cu) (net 2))
 (segment (start 168.25 80.5) (end 168.25 79) (width 0.2032) (layer F.Cu) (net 2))
 (segment (start 168.25 79) (end 167.75 78.5) (width 0.2032) (layer F.Cu) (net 2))
 (segment (start 167.75 78.5) (end 165.808 78.5) (width 0.2032) (layer F.Cu) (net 2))
 (segment (start 165.808 78.5) (end 165.1645 77.8568) (width 0.2032) (layer F.Cu) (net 2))
 (segment (start 186.4 87.4) (end 189 90) (width 0.2032) (layer F.Cu) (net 2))
 (segment (start 189 90) (end 190.1 90) (width 0.2032) (layer F.Cu) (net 2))
 (segment (start 183.2 91.4) (end 185.1 89.5) (width 0.2032) (layer B.Cu) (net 2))
 (segment (start 185.1 89.5) (end 185.1 88.7) (width 0.2032) (layer B.Cu) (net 2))
 (segment (start 185.1 88.7) (end 186.4 87.4) (width 0.2032) (layer B.Cu) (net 2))
 (segment (start 182 92.3) (end 182.3 92.3) (width 0.2032) (layer F.Cu) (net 2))
 (segment (start 182.3 92.3) (end 183.2 91.4) (width 0.2032) (layer F.Cu) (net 2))
 (segment (start 177 82.6) (end 177.2 82.8) (width 0.2032) (layer F.Cu) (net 2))
 (segment (start 177.2 82.8) (end 184.4 82.8) (width 0.2032) (layer F.Cu) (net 2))
 (segment (start 184.4 82.8) (end 186.2 84.6) (width 0.2032) (layer F.Cu) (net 2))
 (segment (start 186.2 84.6) (end 186.4 84.6) (width 0.2032) (layer F.Cu) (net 2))
 (segment (start 173.2 83.2) (end 173.8 82.6) (width 0.2032) (layer B.Cu) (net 2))
 (segment (start 173.8 82.6) (end 177 82.6) (width 0.2032) (layer B.Cu) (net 2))
 (segment (start 186.4 87.4) (end 186.4 84.6) (width 0.2032) (layer B.Cu) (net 2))
 (via (at 186.4 87.4) (size 0.889) (layers F.Cu B.Cu) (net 2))
 (via (at 183.2 91.4) (size 0.889) (layers F.Cu B.Cu) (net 2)) (via (at 177 82.6) (size 0.889) (layers F.Cu B.Cu) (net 2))
 (via (at 173.2 83.2) (size 0.889) (layers F.Cu B.Cu) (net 2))
 (via (at 186.4 84.6) (size 0.889) (layers F.Cu B.Cu) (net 2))
 (segment (start 169.6012 79.7538) (end 169.601 79.7536) (width 0.254) (layer F.Cu) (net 5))
 (segment (start 186.4 88.8) (end 176.2 88.8) (width 0.254) (layer F.Cu) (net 5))
 (segment (start 176.2 88.8) (end 176 88.6) (width 0.254) (layer F.Cu) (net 5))
 (segment (start 176 88.6) (end 176 84.6) (width 0.254) (layer F.Cu) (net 5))
 (segment (start 176 84.6) (end 173.4 82) (width 0.254) (layer F.Cu) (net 5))
 (segment (start 173.4 82) (end 171.848 82) (width 0.254) (layer F.Cu) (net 5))
 (segment (start 171.848 82) (end 169.6012 79.7538) (width 0.254) (layer F.Cu) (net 5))
 (segment (start 169.601 79.754) (end 169.6012 79.7538) (width 0.254) (layer F.Cu) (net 5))
 (segment (start 158.9 104) (end 161.51 104) (width 0.254) (layer F.Cu) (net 5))
 (segment (start 161.51 104) (end 162.56 102.95) (width 0.254) (layer F.Cu) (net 5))
 (segment (start 184.4 94.7) (end 186.3 94.7) (width 0.254) (layer F.Cu) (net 5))
 (segment (start 186.3 94.7) (end 186.4 94.8) (width 0.254) (layer F.Cu) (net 5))
 (segment (start 162.56 102.95) (end 163.45 102.95) (width 0.254) (layer F.Cu) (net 5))
 (segment (start 163.45 102.95) (end 165.6 100.8) (width 0.254) (layer F.Cu) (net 5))
 (segment (start 165.6 100.8) (end 165.6 99.6) (width 0.254) (layer F.Cu) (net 5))
 (segment (start 165.6 99.6) (end 167 98.2) (width 0.254) (layer F.Cu) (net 5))
 (segment (start 167 98.2) (end 185.6 98.2) (width 0.254) (layer F.Cu) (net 5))
 (segment (start 185.6 98.2) (end 186.4 97.4) (width 0.254) (layer B.Cu) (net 5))
 (segment (start 186.4 97.4) (end 186.4 94.8) (width 0.254) (layer B.Cu) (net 5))
 (segment (start 186.4 94.8) (end 186.4 88.8) (width 0.254) (layer B.Cu) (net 5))
 (via (at 186.4 94.8) (size 0.889) (layers F.Cu B.Cu) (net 5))
 (via (at 185.6 98.2) (size 0.889) (layers F.Cu B.Cu) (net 5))
 (via (at 186.4 88.8) (size 0.889) (layers F.Cu B.Cu) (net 5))
 (segment (start 167.3295 77.4818) (end 167.3288 77.4818) (width 0.2032) (layer F.Cu) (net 4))
 (segment (start 167.3288 77.4818) (end 167.061 77.214) (width 0.2032) (layer F.Cu) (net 4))
 (segment (start 167.3295 77.4818) (end 167.061 77.2136) (width 0.2032) (layer F.Cu) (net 4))
 (segment (start 190.1 88) (end 188.5 86.4) (width 0.2032) (layer F.Cu) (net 4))
 (segment (start 188.5 86.4) (end 179.2 86.4) (width 0.2032) (layer F.Cu) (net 4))
 (segment (start 179.2 86.4) (end 178.4 85.6) (width 0.2032) (layer F.Cu) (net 4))
 (segment (start 178.4 85.6) (end 178.4 84) (width 0.2032) (layer F.Cu) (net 4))
 (segment (start 178.4 84) (end 178 83.6) (width 0.2032) (layer F.Cu) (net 4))
 (segment (start 178 83.6) (end 176.4 83.6) (width 0.2032) (layer F.Cu) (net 4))
 (segment (start 176.4 83.6) (end 173.4 80.6) (width 0.2032) (layer F.Cu) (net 4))
 (segment (start 173.4 80.6) (end 173.4 78.8) (width 0.2032) (layer F.Cu) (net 4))
 (segment (start 173.4 78.8) (end 173 78.4) (width 0.2032) (layer F.Cu) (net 4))
 (segment (start 173 78.4) (end 168.65 78.4) (width 0.2032) (layer F.Cu) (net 4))
 (segment (start 168.65 78.4) (end 168 77.75) (width 0.2032) (layer F.Cu) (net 4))
 (segment (start 168 77.75) (end 167.598 77.75) (width 0.2032) (layer F.Cu) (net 4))
 (segment (start 167.598 77.75) (end 167.3295 77.4818) (width 0.2032) (layer F.Cu) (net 4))
 (segment (start 184.4 92.3) (end 187.2 92.3) (width 0.2032) (layer F.Cu) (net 4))
 (segment (start 187.2 92.3) (end 187.5 92.6) (width 0.2032) (layer F.Cu) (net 4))
 (segment (start 187.5 92.6) (end 188.2 91.9) (width 0.2032) (layer B.Cu) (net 4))
 (segment (start 188.2 91.9) (end 188.2 89.9) (width 0.2032) (layer B.Cu) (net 4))
 (segment (start 188.2 89.9) (end 190.1 88) (width 0.2032) (layer B.Cu) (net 4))
 (via (at 187.5 92.6) (size 0.889) (layers F.Cu B.Cu) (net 4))
 (segment (start 190.1 100) (end 197.65 100) (width 0.254) (layer F.Cu) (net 9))
 (segment (start 197.65 100) (end 198.65 101) (width 0.254) (layer F.Cu) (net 9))
 (segment (start 174.8 89.9) (end 174.9 89.9) (width 0.254) (layer F.Cu) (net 9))
 (segment (start 174.9 89.9) (end 176 91) (width 0.254) (layer F.Cu) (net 9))
 (segment (start 176 91) (end 182.5 91) (width 0.254) (layer F.Cu) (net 9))
 (segment (start 182.5 91) (end 183 90.5) (width 0.254) (layer F.Cu) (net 9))
 (segment (start 183 90.5) (end 183.5 90.5) (width 0.254) (layer F.Cu) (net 9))
 (segment (start 183.5 90.5) (end 184 91) (width 0.254) (layer F.Cu) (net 9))
 (segment (start 184 91) (end 187.6 91) (width 0.254) (layer F.Cu) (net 9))
 (segment (start 187.6 91) (end 188.4 91.8) (width 0.254) (layer F.Cu) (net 9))
 (segment (start 188.4 91.8) (end 188.4 98.3) (width 0.254) (layer F.Cu) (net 9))
 (segment (start 188.4 98.3) (end 190.1 100) (width 0.254) (layer F.Cu) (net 9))
 (segment (start 174.8 87.5) (end 174.8 87.6) (width 0.254) (layer F.Cu) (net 10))
 (segment (start 174.8 87.6) (end 173.6 88.8) (width 0.254) (layer F.Cu) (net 10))
 (segment (start 173.6 88.8) (end 173.6 93) (width 0.254) (layer F.Cu) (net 10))
 (segment (start 173.6 93) (end 174.2 93.6) (width 0.254) (layer F.Cu) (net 10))
 (segment (start 174.2 93.6) (end 187.2 93.6) (width 0.254) (layer F.Cu) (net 10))
 (segment (start 187.2 93.6) (end 187.6 94) (width 0.254) (layer F.Cu) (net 10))
 (segment (start 187.6 94) (end 187.6 99.5) (width 0.254) (layer F.Cu) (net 10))
 (segment (start 187.6 99.5) (end 190.1 102) (width 0.254) (layer F.Cu) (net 10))
 (segment (start 190.1 102) (end 197.15 102) (width 0.254) (layer F.Cu) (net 10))
 (segment (start 197.15 102) (end 198.65 103.5) (width 0.254) (layer F.Cu) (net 10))
 (segment (start 174.8 85.1) (end 174.7 85.1) (width 0.254) (layer F.Cu) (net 11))
 (segment (start 174.7 85.1) (end 173.4 86.4) (width 0.254) (layer F.Cu) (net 11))
 (segment (start 173.4 86.4) (end 171.6 86.4) (width 0.254) (layer F.Cu) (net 11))
 (segment (start 171.6 86.4) (end 171.2 86.8) (width 0.254) (layer F.Cu) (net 11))
 (segment (start 171.2 86.8) (end 171.2 95.4) (width 0.254) (layer F.Cu) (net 11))
 (segment (start 171.2 95.4) (end 171.8 96) (width 0.254) (layer F.Cu) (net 11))
 (segment (start 171.8 96) (end 186.292 96) (width 0.254) (layer F.Cu) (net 11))
 (segment (start 186.292 96) (end 186.8 96.508) (width 0.254) (layer F.Cu) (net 11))
 (segment (start 186.8 96.508) (end 186.8 100.7) (width 0.254) (layer F.Cu) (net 11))
 (segment (start 186.8 100.7) (end 190.1 104) (width 0.254) (layer F.Cu) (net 11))
 (segment (start 190.1 104) (end 196.65 104) (width 0.254) (layer F.Cu) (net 11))
 (segment (start 196.65 104) (end 198.65 106) (width 0.254) (layer F.Cu) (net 11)))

